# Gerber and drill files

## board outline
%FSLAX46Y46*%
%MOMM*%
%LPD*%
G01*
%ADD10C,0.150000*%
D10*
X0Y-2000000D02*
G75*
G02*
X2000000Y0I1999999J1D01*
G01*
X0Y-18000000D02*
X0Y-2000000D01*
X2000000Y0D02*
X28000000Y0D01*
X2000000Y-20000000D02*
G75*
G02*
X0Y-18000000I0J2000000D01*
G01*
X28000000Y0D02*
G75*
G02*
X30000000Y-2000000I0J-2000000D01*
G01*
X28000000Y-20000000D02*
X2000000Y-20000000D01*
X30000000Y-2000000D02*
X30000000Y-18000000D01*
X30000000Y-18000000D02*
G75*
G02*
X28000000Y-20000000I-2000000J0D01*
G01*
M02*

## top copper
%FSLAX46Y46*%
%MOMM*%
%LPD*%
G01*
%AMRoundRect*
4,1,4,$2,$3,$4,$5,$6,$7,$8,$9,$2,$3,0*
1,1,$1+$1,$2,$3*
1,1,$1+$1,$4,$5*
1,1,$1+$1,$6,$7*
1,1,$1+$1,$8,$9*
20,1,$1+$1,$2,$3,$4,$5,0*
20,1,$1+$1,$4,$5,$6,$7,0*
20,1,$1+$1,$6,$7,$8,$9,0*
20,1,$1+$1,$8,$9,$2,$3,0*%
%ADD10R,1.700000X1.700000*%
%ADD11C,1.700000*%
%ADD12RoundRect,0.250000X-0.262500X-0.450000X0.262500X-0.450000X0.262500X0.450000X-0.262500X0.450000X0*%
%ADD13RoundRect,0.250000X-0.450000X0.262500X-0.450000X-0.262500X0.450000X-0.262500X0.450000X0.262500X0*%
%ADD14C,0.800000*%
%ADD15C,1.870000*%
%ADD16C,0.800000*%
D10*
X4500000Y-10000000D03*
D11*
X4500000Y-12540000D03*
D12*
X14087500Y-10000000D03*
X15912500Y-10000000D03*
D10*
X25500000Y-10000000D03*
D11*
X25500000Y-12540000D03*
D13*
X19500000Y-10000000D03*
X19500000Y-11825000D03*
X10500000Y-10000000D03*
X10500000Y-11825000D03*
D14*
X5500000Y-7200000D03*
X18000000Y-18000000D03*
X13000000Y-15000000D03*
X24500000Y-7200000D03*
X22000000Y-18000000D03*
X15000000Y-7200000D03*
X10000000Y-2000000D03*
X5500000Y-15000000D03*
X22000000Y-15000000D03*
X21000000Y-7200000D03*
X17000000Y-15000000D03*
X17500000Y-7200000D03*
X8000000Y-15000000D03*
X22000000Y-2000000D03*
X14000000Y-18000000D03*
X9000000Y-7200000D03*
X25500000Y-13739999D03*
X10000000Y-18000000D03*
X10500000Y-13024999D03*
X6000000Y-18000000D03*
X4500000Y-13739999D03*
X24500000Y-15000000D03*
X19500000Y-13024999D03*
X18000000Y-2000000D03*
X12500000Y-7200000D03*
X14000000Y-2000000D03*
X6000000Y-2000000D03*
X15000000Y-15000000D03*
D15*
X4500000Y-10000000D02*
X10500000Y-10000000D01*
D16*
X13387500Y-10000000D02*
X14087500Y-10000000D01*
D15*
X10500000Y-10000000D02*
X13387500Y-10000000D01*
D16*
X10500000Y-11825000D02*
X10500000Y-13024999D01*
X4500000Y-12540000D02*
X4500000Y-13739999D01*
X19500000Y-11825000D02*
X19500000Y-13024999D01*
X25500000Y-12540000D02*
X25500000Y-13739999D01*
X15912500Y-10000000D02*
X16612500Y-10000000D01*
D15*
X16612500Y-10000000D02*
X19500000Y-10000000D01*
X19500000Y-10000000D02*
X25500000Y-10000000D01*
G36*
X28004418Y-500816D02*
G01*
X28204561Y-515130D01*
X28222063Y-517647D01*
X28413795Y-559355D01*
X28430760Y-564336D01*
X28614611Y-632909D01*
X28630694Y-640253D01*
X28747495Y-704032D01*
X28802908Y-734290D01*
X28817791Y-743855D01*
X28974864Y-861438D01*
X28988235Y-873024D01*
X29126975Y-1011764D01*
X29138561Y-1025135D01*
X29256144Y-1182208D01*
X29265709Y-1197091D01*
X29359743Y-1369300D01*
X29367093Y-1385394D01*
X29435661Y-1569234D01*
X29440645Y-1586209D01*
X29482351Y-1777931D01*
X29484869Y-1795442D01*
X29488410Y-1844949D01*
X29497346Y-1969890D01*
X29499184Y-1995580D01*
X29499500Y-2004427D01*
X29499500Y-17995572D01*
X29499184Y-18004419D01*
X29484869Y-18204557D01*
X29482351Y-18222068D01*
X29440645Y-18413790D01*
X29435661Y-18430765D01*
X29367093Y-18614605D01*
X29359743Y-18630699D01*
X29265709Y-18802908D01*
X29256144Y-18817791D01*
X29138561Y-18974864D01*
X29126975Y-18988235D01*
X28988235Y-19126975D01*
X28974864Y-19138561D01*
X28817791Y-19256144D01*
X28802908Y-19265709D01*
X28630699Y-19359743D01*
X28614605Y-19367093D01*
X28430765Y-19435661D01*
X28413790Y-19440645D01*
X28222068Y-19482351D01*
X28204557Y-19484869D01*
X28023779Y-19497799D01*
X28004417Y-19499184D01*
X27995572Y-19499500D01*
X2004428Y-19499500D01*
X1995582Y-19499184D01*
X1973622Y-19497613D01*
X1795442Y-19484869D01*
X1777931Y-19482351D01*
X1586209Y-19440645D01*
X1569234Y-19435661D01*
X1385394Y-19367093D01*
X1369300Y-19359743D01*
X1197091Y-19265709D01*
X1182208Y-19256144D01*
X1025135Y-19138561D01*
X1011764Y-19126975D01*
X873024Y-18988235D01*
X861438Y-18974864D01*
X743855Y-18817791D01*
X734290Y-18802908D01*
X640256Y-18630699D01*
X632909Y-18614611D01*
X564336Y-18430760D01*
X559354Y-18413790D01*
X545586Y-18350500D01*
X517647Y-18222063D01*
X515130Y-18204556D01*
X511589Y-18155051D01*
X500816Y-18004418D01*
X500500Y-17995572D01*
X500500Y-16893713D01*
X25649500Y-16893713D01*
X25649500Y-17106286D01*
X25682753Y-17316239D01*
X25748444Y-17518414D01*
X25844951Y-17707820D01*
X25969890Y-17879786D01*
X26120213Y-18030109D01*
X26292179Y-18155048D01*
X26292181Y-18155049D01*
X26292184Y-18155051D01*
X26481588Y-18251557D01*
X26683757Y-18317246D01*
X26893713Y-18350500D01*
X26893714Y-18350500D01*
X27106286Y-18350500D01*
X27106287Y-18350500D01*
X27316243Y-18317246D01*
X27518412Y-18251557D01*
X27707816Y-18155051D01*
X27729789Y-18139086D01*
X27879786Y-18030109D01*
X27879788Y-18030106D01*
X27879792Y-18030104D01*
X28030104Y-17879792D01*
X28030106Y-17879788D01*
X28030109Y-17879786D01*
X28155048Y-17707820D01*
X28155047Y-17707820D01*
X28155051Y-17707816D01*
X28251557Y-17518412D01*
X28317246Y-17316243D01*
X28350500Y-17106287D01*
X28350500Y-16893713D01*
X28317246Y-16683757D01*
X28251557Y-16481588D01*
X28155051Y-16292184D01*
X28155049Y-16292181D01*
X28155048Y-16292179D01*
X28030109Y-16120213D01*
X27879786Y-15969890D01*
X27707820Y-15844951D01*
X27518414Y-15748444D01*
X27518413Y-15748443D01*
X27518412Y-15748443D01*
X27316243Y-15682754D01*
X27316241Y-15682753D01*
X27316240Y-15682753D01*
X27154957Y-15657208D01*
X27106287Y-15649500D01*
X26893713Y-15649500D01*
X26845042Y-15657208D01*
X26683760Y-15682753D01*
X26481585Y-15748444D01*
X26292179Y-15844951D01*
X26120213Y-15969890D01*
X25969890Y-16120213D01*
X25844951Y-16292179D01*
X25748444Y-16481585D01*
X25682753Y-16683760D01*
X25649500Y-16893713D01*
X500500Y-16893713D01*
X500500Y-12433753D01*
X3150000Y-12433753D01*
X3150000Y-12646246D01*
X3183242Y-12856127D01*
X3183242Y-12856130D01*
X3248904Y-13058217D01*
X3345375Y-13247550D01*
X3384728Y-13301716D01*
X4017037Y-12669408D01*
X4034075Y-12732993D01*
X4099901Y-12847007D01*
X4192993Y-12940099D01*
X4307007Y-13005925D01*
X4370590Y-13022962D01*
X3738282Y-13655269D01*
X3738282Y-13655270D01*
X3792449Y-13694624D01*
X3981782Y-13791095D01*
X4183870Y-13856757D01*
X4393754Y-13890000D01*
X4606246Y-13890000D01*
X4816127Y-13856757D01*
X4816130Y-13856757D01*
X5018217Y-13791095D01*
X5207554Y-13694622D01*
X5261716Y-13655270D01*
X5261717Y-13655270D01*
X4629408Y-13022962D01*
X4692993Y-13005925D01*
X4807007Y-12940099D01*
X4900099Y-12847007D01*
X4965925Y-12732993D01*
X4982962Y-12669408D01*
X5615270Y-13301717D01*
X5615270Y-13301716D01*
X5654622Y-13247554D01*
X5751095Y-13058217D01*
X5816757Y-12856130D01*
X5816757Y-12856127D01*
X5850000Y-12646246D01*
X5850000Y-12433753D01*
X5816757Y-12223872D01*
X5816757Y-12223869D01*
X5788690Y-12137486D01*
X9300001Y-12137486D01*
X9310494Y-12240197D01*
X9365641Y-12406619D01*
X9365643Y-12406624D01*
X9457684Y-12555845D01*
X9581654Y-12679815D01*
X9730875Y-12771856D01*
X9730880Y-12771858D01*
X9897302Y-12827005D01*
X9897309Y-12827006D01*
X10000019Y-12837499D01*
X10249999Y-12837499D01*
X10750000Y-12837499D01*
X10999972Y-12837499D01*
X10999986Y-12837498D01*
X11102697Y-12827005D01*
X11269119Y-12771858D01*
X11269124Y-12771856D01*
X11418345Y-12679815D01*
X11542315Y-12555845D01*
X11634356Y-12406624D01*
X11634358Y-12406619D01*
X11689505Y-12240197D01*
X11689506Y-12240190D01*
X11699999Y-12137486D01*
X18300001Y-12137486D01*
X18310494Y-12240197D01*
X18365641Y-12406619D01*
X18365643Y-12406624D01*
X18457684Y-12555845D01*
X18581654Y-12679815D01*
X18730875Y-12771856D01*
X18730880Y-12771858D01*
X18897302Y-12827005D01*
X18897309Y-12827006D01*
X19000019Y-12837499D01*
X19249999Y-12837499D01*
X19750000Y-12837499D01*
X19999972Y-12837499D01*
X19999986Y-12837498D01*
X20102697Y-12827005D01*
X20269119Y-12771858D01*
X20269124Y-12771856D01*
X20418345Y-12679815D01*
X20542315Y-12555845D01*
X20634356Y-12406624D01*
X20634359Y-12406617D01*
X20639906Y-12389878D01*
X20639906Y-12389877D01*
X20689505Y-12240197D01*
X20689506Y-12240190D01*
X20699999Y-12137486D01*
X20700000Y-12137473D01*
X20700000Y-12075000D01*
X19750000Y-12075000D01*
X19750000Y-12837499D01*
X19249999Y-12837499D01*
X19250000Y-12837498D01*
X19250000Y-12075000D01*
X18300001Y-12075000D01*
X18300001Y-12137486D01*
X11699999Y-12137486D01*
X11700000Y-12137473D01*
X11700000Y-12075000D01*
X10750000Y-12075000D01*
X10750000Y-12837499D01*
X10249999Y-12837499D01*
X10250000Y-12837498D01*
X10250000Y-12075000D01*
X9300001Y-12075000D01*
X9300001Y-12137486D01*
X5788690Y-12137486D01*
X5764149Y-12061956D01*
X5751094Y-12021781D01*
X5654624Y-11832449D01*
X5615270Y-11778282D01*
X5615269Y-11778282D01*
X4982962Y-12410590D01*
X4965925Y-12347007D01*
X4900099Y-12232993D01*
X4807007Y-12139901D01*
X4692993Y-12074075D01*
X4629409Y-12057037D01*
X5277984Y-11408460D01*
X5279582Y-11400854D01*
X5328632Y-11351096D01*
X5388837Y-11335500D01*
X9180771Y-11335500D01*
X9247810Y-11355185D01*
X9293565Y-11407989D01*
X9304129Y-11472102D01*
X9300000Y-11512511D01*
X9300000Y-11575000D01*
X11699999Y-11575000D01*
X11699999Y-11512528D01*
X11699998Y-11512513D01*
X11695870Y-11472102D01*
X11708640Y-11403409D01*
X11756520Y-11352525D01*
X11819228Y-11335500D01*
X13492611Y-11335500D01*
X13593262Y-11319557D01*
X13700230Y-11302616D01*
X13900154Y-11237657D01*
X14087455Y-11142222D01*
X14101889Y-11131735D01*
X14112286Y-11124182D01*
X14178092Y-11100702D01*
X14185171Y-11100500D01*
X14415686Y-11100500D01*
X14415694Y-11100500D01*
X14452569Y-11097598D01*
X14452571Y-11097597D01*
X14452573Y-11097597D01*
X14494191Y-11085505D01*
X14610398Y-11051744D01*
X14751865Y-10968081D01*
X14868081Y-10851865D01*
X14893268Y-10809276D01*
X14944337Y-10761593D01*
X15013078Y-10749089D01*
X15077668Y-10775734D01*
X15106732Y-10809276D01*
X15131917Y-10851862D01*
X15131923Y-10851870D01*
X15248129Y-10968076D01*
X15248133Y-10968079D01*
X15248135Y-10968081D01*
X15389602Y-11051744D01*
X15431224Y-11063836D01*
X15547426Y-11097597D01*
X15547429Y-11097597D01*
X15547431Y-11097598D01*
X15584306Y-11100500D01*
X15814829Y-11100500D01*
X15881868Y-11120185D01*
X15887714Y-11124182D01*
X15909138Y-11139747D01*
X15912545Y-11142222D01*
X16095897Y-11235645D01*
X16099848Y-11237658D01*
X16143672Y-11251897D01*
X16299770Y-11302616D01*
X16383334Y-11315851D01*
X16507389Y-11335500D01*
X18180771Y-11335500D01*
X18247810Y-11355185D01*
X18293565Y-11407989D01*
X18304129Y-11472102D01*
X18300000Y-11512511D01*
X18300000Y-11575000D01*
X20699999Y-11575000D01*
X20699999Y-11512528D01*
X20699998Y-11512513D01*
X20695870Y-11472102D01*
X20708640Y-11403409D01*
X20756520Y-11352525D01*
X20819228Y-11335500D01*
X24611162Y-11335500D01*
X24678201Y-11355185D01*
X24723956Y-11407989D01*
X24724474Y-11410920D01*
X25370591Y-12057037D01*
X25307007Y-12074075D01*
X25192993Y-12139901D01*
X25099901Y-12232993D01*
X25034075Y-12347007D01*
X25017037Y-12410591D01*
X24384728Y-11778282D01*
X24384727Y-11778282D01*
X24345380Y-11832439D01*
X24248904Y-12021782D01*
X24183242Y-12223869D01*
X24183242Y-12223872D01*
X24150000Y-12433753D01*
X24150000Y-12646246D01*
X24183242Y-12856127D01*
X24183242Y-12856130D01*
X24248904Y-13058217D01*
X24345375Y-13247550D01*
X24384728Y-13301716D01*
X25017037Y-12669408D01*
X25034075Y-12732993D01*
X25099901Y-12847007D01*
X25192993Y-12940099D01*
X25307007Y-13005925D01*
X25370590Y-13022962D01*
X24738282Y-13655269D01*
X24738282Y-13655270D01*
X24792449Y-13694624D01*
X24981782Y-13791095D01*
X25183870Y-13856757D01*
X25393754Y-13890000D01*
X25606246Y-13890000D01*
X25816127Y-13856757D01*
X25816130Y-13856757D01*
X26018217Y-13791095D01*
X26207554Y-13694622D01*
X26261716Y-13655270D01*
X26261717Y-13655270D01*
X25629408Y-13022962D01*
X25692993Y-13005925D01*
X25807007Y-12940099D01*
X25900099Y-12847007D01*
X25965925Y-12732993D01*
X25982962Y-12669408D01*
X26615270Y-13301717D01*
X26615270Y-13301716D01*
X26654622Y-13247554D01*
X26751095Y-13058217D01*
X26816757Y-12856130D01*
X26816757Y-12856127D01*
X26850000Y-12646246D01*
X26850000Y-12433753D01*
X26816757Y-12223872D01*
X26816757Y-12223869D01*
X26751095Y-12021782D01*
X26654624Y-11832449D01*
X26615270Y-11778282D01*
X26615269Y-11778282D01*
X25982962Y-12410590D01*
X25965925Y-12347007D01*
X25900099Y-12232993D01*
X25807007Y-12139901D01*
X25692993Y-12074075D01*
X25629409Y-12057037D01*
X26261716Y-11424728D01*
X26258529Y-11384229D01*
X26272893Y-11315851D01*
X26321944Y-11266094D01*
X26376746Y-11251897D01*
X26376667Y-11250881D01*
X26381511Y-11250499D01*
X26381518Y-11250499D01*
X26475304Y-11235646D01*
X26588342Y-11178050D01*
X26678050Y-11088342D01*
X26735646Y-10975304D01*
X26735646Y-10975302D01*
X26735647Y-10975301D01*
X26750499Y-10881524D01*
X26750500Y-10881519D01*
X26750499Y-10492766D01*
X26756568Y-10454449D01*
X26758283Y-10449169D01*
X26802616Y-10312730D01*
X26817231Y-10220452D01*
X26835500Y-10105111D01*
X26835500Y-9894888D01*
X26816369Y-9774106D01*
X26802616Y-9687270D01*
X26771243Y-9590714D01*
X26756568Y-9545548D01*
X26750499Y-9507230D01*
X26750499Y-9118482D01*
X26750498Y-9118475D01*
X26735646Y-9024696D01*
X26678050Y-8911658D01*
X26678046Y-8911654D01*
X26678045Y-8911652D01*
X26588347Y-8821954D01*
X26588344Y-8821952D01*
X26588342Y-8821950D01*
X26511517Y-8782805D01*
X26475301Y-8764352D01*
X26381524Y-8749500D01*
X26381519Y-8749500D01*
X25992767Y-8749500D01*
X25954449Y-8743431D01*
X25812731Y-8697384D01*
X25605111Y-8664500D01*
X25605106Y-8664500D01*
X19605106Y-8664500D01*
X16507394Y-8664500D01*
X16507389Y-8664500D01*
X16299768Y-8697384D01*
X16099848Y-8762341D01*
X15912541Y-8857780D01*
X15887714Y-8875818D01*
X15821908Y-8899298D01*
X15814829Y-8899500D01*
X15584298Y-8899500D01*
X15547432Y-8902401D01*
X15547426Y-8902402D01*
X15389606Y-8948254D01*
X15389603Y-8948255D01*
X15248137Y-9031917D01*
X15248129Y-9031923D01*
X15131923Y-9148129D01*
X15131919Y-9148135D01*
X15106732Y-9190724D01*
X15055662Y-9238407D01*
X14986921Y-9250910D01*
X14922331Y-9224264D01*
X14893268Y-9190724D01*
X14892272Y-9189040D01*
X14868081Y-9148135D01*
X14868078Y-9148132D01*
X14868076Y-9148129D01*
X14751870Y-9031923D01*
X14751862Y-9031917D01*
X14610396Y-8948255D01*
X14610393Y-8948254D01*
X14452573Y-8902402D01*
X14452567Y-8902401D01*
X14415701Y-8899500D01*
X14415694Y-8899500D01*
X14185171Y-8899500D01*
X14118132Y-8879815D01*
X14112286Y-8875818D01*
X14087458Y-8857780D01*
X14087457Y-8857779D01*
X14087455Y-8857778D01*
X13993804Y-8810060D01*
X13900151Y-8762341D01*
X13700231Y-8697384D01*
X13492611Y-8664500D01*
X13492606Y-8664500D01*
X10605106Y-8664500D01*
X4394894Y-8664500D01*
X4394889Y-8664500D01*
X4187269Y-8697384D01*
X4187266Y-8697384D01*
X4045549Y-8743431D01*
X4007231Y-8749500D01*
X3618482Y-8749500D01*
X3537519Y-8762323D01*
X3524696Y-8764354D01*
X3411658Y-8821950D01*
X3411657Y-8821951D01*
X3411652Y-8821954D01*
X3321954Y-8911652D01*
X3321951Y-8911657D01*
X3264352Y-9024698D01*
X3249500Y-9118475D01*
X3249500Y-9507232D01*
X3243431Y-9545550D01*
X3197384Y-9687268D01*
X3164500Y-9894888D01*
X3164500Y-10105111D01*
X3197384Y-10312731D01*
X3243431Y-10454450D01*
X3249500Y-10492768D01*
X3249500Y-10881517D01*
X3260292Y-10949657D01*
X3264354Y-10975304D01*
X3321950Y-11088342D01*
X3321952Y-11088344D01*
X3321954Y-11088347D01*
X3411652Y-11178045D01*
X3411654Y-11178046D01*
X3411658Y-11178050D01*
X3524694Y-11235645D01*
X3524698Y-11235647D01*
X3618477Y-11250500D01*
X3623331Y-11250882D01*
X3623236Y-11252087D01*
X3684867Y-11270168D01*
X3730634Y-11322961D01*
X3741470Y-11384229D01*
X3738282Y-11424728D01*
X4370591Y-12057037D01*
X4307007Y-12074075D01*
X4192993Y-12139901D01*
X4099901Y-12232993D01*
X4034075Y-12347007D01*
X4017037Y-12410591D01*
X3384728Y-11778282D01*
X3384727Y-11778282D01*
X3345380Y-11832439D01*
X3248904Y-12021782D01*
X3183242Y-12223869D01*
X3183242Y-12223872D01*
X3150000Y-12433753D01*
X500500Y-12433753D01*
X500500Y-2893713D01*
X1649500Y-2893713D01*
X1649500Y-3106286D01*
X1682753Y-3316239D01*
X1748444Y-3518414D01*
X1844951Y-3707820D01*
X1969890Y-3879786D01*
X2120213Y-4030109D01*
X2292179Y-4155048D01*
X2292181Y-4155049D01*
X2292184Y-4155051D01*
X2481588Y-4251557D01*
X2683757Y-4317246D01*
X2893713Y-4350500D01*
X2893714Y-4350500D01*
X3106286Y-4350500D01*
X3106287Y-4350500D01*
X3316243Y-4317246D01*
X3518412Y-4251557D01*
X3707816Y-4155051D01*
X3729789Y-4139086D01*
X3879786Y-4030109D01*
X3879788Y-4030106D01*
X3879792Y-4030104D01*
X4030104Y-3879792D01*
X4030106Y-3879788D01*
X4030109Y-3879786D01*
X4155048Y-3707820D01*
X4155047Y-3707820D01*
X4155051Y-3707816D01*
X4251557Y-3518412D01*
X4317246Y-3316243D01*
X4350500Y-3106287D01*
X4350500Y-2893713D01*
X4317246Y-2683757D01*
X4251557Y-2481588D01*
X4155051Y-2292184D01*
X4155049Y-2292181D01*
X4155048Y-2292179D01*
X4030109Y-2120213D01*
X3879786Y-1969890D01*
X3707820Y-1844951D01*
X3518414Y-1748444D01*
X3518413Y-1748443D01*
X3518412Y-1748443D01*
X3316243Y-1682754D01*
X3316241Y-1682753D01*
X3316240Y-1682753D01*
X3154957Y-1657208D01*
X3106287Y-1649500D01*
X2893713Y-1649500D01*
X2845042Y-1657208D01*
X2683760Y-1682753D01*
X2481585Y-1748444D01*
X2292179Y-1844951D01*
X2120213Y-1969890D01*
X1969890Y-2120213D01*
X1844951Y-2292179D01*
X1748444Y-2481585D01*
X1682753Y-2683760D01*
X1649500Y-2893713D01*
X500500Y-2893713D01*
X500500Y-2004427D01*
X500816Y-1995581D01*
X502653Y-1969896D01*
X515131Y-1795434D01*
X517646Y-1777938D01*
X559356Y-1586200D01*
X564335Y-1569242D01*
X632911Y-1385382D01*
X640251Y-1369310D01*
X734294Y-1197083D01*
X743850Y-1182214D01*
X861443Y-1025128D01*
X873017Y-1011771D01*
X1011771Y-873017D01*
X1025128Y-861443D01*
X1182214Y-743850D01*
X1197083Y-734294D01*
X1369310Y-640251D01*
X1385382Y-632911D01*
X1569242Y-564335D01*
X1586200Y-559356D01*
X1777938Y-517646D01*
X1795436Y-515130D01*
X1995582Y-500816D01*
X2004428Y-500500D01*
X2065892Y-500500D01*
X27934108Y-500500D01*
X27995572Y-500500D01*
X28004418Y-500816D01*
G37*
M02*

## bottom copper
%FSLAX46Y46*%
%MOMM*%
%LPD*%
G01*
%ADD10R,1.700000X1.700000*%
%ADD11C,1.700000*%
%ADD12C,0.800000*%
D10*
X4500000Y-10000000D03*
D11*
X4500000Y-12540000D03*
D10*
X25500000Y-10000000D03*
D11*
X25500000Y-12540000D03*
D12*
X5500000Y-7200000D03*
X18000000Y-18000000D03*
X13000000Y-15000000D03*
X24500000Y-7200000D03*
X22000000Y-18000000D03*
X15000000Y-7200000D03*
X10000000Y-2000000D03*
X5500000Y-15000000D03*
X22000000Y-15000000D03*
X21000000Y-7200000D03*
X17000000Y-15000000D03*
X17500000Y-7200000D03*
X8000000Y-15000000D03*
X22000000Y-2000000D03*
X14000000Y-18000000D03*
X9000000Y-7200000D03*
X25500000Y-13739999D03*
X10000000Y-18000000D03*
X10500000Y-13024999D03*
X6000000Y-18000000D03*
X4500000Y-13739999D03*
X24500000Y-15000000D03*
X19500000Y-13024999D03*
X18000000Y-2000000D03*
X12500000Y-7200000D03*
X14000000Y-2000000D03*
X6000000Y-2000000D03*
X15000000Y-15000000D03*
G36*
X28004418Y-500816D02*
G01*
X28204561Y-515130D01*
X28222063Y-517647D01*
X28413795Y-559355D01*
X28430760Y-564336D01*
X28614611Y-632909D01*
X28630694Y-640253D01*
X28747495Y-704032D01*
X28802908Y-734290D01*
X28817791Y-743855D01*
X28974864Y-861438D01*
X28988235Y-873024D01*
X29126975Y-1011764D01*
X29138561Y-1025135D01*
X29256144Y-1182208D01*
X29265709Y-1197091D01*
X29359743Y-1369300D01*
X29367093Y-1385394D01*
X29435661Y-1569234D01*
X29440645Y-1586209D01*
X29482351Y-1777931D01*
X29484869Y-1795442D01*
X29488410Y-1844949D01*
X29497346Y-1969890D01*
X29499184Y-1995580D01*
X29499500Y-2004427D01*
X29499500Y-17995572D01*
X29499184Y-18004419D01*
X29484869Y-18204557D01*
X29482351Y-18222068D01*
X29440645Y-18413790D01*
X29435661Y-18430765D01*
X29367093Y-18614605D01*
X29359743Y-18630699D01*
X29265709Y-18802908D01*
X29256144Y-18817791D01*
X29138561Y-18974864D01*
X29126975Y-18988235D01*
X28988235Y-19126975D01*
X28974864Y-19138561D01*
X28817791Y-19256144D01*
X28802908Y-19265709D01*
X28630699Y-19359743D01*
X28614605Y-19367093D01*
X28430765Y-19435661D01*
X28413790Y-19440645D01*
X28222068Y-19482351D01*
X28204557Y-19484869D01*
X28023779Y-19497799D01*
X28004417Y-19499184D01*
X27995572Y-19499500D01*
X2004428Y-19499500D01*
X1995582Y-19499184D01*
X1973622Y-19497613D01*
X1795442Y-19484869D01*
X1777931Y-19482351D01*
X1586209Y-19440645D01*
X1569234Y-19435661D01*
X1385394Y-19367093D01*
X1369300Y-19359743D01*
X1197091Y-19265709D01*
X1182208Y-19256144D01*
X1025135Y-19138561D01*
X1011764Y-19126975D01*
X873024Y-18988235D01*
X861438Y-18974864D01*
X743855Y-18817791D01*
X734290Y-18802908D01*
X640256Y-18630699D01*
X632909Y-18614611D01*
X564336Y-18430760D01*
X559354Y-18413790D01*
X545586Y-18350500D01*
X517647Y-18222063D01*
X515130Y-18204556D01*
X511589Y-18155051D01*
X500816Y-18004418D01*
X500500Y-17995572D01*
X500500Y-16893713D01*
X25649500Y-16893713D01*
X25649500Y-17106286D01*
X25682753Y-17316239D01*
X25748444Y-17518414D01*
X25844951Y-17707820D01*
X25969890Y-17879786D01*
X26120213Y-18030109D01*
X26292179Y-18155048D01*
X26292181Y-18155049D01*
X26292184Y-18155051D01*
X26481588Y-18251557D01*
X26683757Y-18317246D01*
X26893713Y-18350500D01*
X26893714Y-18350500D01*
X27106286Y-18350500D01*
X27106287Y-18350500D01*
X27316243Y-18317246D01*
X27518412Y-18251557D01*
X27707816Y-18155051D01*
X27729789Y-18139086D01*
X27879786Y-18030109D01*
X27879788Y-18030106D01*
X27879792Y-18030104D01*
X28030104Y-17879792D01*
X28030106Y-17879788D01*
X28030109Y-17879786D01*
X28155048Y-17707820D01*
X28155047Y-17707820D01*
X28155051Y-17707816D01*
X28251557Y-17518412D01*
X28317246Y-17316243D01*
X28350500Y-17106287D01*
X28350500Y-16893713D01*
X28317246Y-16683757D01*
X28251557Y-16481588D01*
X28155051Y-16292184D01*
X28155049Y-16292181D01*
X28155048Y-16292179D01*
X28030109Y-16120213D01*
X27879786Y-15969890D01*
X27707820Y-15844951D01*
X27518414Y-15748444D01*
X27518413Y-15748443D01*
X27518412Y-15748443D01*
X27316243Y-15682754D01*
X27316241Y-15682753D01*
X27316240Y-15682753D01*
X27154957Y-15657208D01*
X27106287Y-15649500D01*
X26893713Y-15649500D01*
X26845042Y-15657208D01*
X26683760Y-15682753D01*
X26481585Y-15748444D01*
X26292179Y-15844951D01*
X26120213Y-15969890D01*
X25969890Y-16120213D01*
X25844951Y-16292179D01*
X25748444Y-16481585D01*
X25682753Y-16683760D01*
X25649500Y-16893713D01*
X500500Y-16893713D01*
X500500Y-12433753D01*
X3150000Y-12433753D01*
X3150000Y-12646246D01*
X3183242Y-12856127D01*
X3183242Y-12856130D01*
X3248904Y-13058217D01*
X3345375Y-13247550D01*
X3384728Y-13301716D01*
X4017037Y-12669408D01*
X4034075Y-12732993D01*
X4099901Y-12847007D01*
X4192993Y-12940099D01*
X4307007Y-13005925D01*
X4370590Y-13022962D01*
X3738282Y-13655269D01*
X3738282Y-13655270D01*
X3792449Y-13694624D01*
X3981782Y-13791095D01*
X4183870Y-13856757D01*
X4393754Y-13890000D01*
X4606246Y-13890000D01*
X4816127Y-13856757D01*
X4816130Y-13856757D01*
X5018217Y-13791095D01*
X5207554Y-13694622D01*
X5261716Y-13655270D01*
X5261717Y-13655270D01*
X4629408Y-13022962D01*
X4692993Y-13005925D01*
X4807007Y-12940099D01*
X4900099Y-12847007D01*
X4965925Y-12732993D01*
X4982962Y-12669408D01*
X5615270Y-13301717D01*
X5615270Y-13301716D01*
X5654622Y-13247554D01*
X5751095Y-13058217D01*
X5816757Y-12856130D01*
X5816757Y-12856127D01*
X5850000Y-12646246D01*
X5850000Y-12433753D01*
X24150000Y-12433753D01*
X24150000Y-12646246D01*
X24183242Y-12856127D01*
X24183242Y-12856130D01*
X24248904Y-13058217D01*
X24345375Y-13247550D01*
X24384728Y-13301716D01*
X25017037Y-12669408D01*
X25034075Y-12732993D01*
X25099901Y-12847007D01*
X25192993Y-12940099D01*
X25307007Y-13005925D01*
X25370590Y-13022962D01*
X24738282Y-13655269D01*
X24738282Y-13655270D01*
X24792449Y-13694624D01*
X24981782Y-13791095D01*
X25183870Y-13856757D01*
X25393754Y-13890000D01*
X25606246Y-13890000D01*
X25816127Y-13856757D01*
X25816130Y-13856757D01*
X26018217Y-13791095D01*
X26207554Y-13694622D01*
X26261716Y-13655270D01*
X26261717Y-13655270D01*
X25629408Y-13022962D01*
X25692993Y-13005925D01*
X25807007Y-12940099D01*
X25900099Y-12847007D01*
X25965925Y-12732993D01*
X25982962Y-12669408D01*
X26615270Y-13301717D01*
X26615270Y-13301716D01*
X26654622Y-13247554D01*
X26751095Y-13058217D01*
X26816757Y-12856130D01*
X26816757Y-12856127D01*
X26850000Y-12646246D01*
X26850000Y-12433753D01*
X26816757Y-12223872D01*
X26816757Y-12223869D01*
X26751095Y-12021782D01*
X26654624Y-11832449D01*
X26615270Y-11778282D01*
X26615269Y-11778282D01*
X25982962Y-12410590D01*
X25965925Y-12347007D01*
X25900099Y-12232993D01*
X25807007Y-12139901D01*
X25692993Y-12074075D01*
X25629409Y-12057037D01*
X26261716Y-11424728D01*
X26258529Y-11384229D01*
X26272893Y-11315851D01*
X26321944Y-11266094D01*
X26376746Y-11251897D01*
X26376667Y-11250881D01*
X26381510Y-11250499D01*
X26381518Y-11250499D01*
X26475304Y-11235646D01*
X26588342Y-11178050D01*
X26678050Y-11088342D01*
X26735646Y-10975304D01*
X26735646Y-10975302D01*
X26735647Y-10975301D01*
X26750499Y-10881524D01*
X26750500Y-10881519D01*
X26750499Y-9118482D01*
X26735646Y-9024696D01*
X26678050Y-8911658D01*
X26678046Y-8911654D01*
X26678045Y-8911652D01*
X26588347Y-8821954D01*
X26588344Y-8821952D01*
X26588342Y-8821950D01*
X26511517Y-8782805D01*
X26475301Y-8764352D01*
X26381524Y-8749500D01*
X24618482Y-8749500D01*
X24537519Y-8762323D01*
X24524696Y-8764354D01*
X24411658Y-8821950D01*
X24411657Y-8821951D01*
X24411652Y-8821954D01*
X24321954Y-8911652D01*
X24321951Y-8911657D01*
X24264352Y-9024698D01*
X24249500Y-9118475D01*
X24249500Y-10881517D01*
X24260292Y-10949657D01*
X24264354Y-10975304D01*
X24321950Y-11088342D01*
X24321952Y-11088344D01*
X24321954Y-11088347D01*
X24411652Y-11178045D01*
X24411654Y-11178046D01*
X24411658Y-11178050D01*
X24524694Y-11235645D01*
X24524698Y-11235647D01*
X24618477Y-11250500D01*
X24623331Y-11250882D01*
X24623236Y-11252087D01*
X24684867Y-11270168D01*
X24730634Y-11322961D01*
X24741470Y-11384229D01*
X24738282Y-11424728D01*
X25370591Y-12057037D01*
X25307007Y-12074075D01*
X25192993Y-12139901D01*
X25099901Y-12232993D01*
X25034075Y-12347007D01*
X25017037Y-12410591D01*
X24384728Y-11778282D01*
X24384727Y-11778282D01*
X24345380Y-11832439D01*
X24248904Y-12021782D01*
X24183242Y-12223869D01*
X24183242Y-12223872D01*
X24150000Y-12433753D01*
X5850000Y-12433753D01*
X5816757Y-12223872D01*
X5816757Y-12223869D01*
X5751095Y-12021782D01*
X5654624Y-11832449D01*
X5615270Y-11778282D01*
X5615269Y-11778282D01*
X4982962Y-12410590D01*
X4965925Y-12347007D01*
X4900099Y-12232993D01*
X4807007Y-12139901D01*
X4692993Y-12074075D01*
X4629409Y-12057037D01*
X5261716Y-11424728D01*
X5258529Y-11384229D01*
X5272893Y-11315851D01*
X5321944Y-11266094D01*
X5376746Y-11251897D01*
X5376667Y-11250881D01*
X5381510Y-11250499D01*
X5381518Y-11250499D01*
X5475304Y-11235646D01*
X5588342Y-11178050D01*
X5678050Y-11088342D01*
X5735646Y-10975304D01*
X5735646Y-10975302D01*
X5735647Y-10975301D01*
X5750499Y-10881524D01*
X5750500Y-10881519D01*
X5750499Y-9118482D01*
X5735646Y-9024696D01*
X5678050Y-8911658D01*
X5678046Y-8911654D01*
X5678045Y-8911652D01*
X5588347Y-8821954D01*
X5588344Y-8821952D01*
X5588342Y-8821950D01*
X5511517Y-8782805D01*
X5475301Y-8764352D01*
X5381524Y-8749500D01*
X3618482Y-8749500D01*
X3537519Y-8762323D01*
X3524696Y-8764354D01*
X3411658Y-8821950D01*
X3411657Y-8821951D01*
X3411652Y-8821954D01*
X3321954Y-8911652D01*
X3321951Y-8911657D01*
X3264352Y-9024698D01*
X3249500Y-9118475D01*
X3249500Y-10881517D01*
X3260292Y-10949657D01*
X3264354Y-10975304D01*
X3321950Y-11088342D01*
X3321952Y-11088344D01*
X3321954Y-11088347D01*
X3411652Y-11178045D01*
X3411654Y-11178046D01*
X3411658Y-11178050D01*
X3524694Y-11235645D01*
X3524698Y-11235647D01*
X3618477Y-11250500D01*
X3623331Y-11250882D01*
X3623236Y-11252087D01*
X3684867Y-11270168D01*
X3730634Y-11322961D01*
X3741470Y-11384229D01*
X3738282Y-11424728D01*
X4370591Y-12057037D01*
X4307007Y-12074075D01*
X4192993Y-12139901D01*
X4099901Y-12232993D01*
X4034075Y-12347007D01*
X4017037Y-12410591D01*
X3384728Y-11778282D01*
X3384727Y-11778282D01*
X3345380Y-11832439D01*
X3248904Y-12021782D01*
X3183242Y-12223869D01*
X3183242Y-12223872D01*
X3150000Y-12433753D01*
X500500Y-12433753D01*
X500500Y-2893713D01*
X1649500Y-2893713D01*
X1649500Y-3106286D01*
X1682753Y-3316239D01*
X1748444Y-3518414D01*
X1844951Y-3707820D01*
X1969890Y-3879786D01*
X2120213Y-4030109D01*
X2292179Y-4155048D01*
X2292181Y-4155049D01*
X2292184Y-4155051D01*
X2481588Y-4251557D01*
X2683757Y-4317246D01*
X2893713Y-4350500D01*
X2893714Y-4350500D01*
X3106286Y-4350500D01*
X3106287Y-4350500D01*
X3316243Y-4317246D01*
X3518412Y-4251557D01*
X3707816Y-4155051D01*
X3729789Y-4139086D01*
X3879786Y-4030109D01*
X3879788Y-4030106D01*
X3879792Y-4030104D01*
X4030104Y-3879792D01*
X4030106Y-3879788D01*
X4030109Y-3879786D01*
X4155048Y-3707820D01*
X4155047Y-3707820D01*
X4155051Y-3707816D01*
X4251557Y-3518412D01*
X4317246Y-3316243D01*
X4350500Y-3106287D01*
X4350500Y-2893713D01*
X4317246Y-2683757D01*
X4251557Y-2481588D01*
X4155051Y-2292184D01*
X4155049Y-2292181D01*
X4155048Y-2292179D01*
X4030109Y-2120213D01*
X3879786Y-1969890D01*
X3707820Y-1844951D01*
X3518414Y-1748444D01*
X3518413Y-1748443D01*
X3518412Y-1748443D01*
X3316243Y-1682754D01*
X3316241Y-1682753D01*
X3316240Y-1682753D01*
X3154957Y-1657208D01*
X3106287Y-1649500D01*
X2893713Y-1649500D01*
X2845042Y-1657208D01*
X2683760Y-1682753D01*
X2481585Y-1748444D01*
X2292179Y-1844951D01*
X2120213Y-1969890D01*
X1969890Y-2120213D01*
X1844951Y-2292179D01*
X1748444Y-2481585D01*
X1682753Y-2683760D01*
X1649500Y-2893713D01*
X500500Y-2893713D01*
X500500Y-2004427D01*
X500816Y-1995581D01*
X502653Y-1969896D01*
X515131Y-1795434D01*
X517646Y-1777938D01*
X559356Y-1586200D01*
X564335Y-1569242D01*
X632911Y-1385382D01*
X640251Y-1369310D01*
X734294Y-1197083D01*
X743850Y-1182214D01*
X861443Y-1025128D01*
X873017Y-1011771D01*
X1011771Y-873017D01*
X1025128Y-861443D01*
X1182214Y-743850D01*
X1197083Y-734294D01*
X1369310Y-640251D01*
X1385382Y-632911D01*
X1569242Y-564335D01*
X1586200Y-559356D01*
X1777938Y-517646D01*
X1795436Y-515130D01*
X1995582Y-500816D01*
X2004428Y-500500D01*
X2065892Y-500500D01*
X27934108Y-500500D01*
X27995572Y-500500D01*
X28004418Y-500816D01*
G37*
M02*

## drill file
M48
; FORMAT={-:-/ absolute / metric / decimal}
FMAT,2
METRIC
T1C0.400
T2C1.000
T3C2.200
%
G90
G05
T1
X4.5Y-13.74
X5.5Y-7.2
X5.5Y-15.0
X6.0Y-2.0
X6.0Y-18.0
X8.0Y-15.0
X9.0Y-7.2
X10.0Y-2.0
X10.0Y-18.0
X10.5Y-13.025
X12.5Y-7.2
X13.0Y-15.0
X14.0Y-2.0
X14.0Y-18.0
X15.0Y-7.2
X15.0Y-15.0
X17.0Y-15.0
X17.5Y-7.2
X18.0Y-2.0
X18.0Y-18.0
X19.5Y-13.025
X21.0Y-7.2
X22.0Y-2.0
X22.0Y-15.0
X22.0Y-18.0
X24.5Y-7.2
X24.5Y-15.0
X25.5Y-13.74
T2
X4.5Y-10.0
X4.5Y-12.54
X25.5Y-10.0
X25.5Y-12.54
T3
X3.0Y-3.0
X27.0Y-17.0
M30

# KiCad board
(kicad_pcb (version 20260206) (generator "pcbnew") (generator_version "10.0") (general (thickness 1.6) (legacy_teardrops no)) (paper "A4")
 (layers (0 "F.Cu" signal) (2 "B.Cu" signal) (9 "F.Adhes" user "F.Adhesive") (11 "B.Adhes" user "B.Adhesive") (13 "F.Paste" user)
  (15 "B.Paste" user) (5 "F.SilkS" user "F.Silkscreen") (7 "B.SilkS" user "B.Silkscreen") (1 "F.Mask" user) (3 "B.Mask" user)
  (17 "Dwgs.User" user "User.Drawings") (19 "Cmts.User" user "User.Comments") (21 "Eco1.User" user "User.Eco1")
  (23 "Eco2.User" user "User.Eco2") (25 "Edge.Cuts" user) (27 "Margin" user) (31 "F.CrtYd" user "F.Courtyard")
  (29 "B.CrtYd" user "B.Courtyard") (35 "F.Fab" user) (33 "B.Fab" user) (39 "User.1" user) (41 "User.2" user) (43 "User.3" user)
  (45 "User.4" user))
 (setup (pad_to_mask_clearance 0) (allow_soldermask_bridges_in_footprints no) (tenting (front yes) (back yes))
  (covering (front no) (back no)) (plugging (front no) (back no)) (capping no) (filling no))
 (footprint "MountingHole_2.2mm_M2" (layer "F.Cu") (at 3 3)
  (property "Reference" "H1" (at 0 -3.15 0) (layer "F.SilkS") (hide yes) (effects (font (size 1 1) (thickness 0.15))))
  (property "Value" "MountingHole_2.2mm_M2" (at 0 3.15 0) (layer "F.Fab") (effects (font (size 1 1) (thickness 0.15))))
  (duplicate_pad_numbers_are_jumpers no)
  (pad "" np_thru_hole circle (at 0 0) (size 2.2 2.2) (drill 2.2) (layers "*.Cu" "*.Mask")))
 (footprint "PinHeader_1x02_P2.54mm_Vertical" (layer "F.Cu") (at 4.5 10)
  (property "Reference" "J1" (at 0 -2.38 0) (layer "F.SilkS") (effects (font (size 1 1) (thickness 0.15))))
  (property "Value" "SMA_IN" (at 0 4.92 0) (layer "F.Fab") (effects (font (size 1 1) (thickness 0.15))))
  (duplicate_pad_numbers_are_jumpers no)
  (pad "1" thru_hole rect (at 0 0) (size 1.7 1.7) (drill 1) (layers "*.Cu" "*.Mask") (remove_unused_layers no) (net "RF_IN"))
  (pad "2" thru_hole circle (at 0 2.54) (size 1.7 1.7) (drill 1) (layers "*.Cu" "*.Mask") (remove_unused_layers no) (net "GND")))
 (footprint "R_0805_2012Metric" (layer "F.Cu") (at 15 10)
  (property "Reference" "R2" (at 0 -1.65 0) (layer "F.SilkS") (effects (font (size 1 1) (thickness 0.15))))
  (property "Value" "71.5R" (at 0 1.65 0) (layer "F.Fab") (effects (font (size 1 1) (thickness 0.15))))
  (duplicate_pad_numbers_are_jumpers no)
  (pad "1" smd roundrect (at -0.9125 0) (size 1.025 1.4) (layers "F.Cu" "F.Mask" "F.Paste") (roundrect_rratio 0.243902) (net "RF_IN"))
  (pad "2" smd roundrect (at 0.9125 0) (size 1.025 1.4) (layers "F.Cu" "F.Mask" "F.Paste") (roundrect_rratio 0.243902) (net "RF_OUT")))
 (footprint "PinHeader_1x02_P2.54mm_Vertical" (layer "F.Cu") (at 25.5 10)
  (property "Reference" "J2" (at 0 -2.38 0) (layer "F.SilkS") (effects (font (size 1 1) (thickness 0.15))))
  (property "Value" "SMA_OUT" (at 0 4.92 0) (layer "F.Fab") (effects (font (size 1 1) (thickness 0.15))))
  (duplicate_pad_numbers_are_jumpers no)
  (pad "1" thru_hole rect (at 0 0) (size 1.7 1.7) (drill 1) (layers "*.Cu" "*.Mask") (remove_unused_layers no) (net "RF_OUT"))
  (pad "2" thru_hole circle (at 0 2.54) (size 1.7 1.7) (drill 1) (layers "*.Cu" "*.Mask") (remove_unused_layers no) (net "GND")))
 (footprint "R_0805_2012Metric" (layer "F.Cu") (at 19.5 10.9125 -90)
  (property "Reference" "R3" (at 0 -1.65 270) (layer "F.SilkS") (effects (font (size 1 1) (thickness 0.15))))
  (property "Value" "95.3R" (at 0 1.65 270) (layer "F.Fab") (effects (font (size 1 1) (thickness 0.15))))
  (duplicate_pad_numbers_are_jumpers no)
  (pad "1" smd roundrect (at -0.9125 0 270) (size 1.025 1.4) (layers "F.Cu" "F.Mask" "F.Paste") (roundrect_rratio 0.243902) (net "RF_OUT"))
  (pad "2" smd roundrect (at 0.9125 0 270) (size 1.025 1.4) (layers "F.Cu" "F.Mask" "F.Paste") (roundrect_rratio 0.243902) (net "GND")))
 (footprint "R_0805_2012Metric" (layer "F.Cu") (at 10.5 10.9125 -90)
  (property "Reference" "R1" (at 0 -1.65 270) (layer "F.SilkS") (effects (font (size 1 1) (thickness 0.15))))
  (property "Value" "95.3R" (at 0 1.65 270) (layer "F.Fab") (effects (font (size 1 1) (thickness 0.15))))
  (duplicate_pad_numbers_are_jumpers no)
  (pad "1" smd roundrect (at -0.9125 0 270) (size 1.025 1.4) (layers "F.Cu" "F.Mask" "F.Paste") (roundrect_rratio 0.243902) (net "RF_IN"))
  (pad "2" smd roundrect (at 0.9125 0 270) (size 1.025 1.4) (layers "F.Cu" "F.Mask" "F.Paste") (roundrect_rratio 0.243902) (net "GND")))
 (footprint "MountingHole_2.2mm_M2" (layer "F.Cu") (at 27 17)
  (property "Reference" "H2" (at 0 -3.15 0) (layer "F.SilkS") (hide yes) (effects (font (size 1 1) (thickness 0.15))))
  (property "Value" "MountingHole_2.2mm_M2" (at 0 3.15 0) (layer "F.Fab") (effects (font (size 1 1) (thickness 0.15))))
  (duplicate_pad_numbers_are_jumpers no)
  (pad "" np_thru_hole circle (at 0 0) (size 2.2 2.2) (drill 2.2) (layers "*.Cu" "*.Mask")))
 (gr_arc (start 0 2) (mid 0.585786 0.585786) (end 2 0) (stroke (width 0.15) (type default)) (layer "Edge.Cuts"))
 (gr_line (start 0 18) (end 0 2) (stroke (width 0.15) (type default)) (layer "Edge.Cuts"))
 (gr_line (start 2 0) (end 28 0) (stroke (width 0.15) (type default)) (layer "Edge.Cuts"))
 (gr_arc (start 2 20) (mid 0.585786 19.414214) (end 0 18) (stroke (width 0.15) (type default)) (layer "Edge.Cuts"))
 (gr_arc (start 28 0) (mid 29.414214 0.585786) (end 30 2) (stroke (width 0.15) (type default)) (layer "Edge.Cuts"))
 (gr_line (start 28 20) (end 2 20) (stroke (width 0.15) (type default)) (layer "Edge.Cuts"))
 (gr_line (start 30 2) (end 30 18) (stroke (width 0.15) (type default)) (layer "Edge.Cuts"))
 (gr_arc (start 30 18) (mid 29.414214 19.414214) (end 28 20) (stroke (width 0.15) (type default)) (layer "Edge.Cuts"))
 (segment (start 4.5 10) (end 10.5 10) (width 1.87) (layer "F.Cu") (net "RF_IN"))
 (segment (start 13.3875 10) (end 14.0875 10) (width 0.8) (layer "F.Cu") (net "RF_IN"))
 (segment (start 10.5 10) (end 13.3875 10) (width 1.87) (layer "F.Cu") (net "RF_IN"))
 (segment (start 10.5 11.825) (end 10.5 13.024999) (width 0.8) (layer "F.Cu") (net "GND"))
 (segment (start 4.5 12.54) (end 4.5 13.739999) (width 0.8) (layer "F.Cu") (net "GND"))
 (segment (start 19.5 11.825) (end 19.5 13.024999) (width 0.8) (layer "F.Cu") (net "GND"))
 (segment (start 25.5 12.54) (end 25.5 13.739999) (width 0.8) (layer "F.Cu") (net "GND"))
 (via (at 5.5 7.2) (size 0.8) (drill 0.4) (layers "F.Cu" "B.Cu") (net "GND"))
 (via (at 18 18) (size 0.8) (drill 0.4) (layers "F.Cu" "B.Cu") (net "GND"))
 (via (at 13 15) (size 0.8) (drill 0.4) (layers "F.Cu" "B.Cu") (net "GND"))
 (via (at 24.5 7.2) (size 0.8) (drill 0.4) (layers "F.Cu" "B.Cu") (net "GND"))
 (via (at 22 18) (size 0.8) (drill 0.4) (layers "F.Cu" "B.Cu") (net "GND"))
 (via (at 15 7.2) (size 0.8) (drill 0.4) (layers "F.Cu" "B.Cu") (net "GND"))
 (via (at 10 2) (size 0.8) (drill 0.4) (layers "F.Cu" "B.Cu") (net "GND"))
 (via (at 5.5 15) (size 0.8) (drill 0.4) (layers "F.Cu" "B.Cu") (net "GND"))
 (via (at 22 15) (size 0.8) (drill 0.4) (layers "F.Cu" "B.Cu") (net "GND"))
 (via (at 21 7.2) (size 0.8) (drill 0.4) (layers "F.Cu" "B.Cu") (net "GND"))
 (via (at 17 15) (size 0.8) (drill 0.4) (layers "F.Cu" "B.Cu") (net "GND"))
 (via (at 17.5 7.2) (size 0.8) (drill 0.4) (layers "F.Cu" "B.Cu") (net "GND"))
 (via (at 8 15) (size 0.8) (drill 0.4) (layers "F.Cu" "B.Cu") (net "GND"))
 (via (at 22 2) (size 0.8) (drill 0.4) (layers "F.Cu" "B.Cu") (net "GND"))
 (via (at 14 18) (size 0.8) (drill 0.4) (layers "F.Cu" "B.Cu") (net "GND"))
 (via (at 9 7.2) (size 0.8) (drill 0.4) (layers "F.Cu" "B.Cu") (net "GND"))
 (via (at 25.5 13.739999) (size 0.8) (drill 0.4) (layers "F.Cu" "B.Cu") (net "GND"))
 (via (at 10 18) (size 0.8) (drill 0.4) (layers "F.Cu" "B.Cu") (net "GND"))
 (via (at 10.5 13.024999) (size 0.8) (drill 0.4) (layers "F.Cu" "B.Cu") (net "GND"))
 (via (at 6 18) (size 0.8) (drill 0.4) (layers "F.Cu" "B.Cu") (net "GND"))
 (via (at 4.5 13.739999) (size 0.8) (drill 0.4) (layers "F.Cu" "B.Cu") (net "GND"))
 (via (at 24.5 15) (size 0.8) (drill 0.4) (layers "F.Cu" "B.Cu") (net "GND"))
 (via (at 19.5 13.024999) (size 0.8) (drill 0.4) (layers "F.Cu" "B.Cu") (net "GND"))
 (via (at 18 2) (size 0.8) (drill 0.4) (layers "F.Cu" "B.Cu") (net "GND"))
 (via (at 12.5 7.2) (size 0.8) (drill 0.4) (layers "F.Cu" "B.Cu") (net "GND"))
 (via (at 14 2) (size 0.8) (drill 0.4) (layers "F.Cu" "B.Cu") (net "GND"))
 (via (at 6 2) (size 0.8) (drill 0.4) (layers "F.Cu" "B.Cu") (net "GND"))
 (via (at 15 15) (size 0.8) (drill 0.4) (layers "F.Cu" "B.Cu") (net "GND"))
 (segment (start 15.9125 10) (end 16.6125 10) (width 0.8) (layer "F.Cu") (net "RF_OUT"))
 (segment (start 16.6125 10) (end 19.5 10) (width 1.87) (layer "F.Cu") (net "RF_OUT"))
 (segment (start 19.5 10) (end 25.5 10) (width 1.87) (layer "F.Cu") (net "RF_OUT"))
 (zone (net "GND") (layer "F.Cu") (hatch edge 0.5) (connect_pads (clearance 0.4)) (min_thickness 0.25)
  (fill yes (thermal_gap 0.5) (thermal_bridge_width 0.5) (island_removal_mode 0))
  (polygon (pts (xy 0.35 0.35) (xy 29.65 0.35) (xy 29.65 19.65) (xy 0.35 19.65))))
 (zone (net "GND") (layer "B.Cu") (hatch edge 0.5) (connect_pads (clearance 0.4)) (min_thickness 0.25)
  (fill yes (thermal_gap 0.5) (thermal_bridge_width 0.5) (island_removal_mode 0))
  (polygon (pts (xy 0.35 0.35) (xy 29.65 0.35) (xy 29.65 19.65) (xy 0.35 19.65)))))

